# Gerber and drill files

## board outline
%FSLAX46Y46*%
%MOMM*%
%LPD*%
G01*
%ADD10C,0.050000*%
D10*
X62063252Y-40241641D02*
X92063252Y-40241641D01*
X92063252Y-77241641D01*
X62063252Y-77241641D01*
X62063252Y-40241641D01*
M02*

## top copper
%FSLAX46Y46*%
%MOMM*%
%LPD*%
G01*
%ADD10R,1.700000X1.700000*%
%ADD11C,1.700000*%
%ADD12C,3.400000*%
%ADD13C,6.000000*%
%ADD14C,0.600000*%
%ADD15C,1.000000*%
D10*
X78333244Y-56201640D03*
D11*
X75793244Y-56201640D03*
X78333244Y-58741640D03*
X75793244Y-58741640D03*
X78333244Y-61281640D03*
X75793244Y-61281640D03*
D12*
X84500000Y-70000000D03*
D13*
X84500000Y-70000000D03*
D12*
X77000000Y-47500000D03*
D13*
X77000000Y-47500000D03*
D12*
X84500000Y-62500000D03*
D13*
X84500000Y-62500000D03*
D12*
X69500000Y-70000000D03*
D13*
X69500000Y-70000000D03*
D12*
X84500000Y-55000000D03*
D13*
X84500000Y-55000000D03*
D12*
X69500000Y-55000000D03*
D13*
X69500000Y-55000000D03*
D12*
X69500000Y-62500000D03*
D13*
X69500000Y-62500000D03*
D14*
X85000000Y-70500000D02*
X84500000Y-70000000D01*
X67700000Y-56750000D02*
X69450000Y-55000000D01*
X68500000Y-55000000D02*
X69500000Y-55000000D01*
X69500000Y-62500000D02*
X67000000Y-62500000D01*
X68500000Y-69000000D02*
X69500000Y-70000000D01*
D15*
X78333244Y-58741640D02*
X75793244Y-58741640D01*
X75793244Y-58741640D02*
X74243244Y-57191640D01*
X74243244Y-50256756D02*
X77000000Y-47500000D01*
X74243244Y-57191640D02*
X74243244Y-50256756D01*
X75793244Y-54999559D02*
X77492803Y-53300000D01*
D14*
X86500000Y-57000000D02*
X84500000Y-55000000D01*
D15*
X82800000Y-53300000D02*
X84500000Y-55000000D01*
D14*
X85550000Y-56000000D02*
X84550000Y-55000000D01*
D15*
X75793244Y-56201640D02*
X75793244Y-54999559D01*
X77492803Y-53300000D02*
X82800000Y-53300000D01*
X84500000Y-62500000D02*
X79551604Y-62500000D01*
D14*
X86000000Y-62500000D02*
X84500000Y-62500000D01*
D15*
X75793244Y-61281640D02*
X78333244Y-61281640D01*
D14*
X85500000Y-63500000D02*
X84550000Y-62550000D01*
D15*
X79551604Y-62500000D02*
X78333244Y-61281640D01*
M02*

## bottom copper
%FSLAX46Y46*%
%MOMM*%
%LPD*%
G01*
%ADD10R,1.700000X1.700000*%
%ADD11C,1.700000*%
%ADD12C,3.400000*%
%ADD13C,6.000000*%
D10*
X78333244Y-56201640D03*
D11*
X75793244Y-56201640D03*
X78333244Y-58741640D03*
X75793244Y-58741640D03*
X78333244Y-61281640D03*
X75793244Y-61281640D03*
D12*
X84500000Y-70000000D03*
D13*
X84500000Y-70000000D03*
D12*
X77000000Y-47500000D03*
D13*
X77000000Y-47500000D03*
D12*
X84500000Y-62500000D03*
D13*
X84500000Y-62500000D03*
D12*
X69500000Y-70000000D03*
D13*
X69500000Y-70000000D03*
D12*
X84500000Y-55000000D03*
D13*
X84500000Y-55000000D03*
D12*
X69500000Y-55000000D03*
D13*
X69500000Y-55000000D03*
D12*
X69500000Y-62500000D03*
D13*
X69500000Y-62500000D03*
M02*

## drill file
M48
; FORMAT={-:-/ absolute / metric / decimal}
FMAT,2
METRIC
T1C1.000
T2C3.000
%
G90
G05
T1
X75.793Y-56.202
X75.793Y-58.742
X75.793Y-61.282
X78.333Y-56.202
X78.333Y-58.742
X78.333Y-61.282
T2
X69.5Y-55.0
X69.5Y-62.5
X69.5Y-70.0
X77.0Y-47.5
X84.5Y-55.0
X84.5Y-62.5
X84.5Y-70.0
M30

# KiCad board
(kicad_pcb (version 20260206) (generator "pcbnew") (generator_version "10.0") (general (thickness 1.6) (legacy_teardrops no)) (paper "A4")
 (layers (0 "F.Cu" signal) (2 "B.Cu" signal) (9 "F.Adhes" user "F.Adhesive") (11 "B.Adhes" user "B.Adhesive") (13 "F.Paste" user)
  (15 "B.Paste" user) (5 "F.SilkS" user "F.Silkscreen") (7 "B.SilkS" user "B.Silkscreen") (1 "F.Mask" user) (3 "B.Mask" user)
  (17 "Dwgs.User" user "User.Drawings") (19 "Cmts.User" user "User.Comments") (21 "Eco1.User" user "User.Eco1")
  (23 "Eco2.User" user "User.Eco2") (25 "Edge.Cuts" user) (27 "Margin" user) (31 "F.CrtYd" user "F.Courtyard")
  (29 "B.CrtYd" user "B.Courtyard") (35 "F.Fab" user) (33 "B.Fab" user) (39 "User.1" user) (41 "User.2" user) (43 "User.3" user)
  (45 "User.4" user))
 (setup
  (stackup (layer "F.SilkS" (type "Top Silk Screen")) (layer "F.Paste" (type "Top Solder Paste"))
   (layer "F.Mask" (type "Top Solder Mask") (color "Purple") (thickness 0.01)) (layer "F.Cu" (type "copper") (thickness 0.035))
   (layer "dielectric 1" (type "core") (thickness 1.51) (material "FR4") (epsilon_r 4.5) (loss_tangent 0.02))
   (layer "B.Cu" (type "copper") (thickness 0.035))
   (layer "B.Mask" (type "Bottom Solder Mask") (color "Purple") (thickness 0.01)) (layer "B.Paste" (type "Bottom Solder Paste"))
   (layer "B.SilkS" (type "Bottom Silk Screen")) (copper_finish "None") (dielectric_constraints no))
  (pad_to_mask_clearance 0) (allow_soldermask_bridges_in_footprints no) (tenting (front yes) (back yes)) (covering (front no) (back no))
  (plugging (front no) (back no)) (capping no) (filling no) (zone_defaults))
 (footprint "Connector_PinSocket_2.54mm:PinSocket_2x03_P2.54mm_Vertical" (layer "F.Cu") (at 78.333244 56.20164)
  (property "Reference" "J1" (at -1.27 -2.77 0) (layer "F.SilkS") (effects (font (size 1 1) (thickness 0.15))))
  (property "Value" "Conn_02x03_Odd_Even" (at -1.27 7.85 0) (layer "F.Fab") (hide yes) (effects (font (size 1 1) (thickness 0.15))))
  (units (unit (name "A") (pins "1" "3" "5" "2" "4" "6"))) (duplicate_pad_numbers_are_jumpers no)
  (pad "1" thru_hole rect (at 0 0) (size 1.7 1.7) (drill 1) (layers "*.Cu" "*.Mask") (remove_unused_layers no)
   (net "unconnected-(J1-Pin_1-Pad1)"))
  (pad "2" thru_hole circle (at -2.54 0) (size 1.7 1.7) (drill 1) (layers "*.Cu" "*.Mask") (remove_unused_layers no) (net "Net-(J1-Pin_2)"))
  (pad "3" thru_hole circle (at 0 2.54) (size 1.7 1.7) (drill 1) (layers "*.Cu" "*.Mask") (remove_unused_layers no) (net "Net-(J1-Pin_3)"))
  (pad "4" thru_hole circle (at -2.54 2.54) (size 1.7 1.7) (drill 1) (layers "*.Cu" "*.Mask") (remove_unused_layers no)
   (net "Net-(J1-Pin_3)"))
  (pad "5" thru_hole circle (at 0 5.08) (size 1.7 1.7) (drill 1) (layers "*.Cu" "*.Mask") (remove_unused_layers no) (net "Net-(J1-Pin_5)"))
  (pad "6" thru_hole circle (at -2.54 5.08) (size 1.7 1.7) (drill 1) (layers "*.Cu" "*.Mask") (remove_unused_layers no)
   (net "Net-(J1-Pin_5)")))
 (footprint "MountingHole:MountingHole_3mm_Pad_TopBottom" (layer "F.Cu") (at 84.5 70)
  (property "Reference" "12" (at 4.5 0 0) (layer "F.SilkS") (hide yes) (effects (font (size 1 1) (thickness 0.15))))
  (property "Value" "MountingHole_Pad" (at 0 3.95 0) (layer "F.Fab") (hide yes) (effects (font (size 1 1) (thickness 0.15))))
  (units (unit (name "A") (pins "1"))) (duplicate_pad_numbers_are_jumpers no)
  (pad "1" thru_hole circle (at 0 0) (size 3.4 3.4) (drill 3) (layers "*.Cu" "*.Mask") (remove_unused_layers no)
   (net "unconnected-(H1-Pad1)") (zone_connect 2))
  (pad "1" connect circle (at 0 0) (size 6 6) (layers "F.Cu" "F.Mask") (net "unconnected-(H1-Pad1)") (zone_connect 2))
  (pad "1" connect circle (at 0 0) (size 6 6) (layers "B.Cu" "B.Mask") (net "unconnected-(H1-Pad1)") (zone_connect 2)))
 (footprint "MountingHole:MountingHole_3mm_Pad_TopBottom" (layer "F.Cu") (at 77 47.5)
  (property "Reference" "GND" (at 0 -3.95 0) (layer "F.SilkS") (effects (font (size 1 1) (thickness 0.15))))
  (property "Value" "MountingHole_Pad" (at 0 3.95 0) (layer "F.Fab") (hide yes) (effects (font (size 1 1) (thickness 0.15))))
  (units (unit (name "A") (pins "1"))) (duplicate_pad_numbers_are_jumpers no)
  (pad "1" thru_hole circle (at 0 0) (size 3.4 3.4) (drill 3) (layers "*.Cu" "*.Mask") (remove_unused_layers no) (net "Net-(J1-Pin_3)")
   (zone_connect 2))
  (pad "1" connect circle (at 0 0) (size 6 6) (layers "F.Cu" "F.Mask") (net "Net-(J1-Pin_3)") (zone_connect 2))
  (pad "1" connect circle (at 0 0) (size 6 6) (layers "B.Cu" "B.Mask") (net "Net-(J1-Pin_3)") (zone_connect 2)))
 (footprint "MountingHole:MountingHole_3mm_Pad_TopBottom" (layer "F.Cu") (at 84.5 62.5)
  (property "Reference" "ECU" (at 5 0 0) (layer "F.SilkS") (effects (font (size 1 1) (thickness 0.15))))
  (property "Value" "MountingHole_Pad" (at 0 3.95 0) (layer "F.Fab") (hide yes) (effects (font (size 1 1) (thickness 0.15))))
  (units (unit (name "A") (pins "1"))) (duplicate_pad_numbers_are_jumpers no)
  (pad "1" thru_hole circle (at 0 0) (size 3.4 3.4) (drill 3) (layers "*.Cu" "*.Mask") (remove_unused_layers no) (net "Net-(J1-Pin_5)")
   (zone_connect 2))
  (pad "1" connect circle (at 0 0) (size 6 6) (layers "F.Cu" "F.Mask") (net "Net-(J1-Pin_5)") (zone_connect 2))
  (pad "1" connect circle (at 0 0) (size 6 6) (layers "B.Cu" "B.Mask") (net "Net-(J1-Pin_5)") (zone_connect 2)))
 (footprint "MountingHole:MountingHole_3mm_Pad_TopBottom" (layer "F.Cu") (at 69.5 70)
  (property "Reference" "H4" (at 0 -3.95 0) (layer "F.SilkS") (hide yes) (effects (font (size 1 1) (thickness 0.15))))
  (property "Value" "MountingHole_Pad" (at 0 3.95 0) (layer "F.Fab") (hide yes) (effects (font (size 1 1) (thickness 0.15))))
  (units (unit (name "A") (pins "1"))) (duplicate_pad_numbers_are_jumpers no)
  (pad "1" thru_hole circle (at 0 0) (size 3.4 3.4) (drill 3) (layers "*.Cu" "*.Mask") (remove_unused_layers no)
   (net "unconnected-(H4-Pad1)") (zone_connect 2))
  (pad "1" connect circle (at 0 0) (size 6 6) (layers "F.Cu" "F.Mask") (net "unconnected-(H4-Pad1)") (zone_connect 2))
  (pad "1" connect circle (at 0 0) (size 6 6) (layers "B.Cu" "B.Mask") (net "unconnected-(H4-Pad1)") (zone_connect 2)))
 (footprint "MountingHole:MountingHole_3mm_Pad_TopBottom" (layer "F.Cu") (at 84.5 55)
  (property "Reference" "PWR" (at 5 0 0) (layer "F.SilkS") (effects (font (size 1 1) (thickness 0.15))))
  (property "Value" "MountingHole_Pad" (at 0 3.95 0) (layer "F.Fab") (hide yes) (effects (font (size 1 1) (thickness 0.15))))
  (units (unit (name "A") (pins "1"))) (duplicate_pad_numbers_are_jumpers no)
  (pad "1" thru_hole circle (at 0 0) (size 3.4 3.4) (drill 3) (layers "*.Cu" "*.Mask") (remove_unused_layers no) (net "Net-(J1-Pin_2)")
   (zone_connect 2))
  (pad "1" connect circle (at 0 0) (size 6 6) (layers "F.Cu" "F.Mask") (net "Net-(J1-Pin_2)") (zone_connect 2))
  (pad "1" connect circle (at 0 0) (size 6 6) (layers "B.Cu" "B.Mask") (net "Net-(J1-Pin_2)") (zone_connect 2)))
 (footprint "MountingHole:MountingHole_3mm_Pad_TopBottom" (layer "F.Cu") (at 69.5 55)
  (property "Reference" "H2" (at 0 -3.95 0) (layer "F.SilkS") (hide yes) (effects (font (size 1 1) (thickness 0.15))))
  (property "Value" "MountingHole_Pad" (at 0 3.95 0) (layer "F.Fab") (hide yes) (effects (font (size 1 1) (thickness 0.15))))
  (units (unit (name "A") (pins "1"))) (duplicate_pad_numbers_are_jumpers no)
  (pad "1" thru_hole circle (at 0 0) (size 3.4 3.4) (drill 3) (layers "*.Cu" "*.Mask") (remove_unused_layers no)
   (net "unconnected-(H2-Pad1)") (zone_connect 2))
  (pad "1" connect circle (at 0 0) (size 6 6) (layers "F.Cu" "F.Mask") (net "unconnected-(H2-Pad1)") (zone_connect 2))
  (pad "1" connect circle (at 0 0) (size 6 6) (layers "B.Cu" "B.Mask") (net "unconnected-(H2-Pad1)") (zone_connect 2)))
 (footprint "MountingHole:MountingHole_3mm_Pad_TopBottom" (layer "F.Cu") (at 69.5 62.5)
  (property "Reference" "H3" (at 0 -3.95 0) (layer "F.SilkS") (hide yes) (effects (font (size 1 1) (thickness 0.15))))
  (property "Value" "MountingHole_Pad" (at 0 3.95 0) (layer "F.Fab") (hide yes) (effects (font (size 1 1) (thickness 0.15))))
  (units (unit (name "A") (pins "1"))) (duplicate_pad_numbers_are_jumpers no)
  (pad "1" thru_hole circle (at 0 0) (size 3.4 3.4) (drill 3) (layers "*.Cu" "*.Mask") (remove_unused_layers no)
   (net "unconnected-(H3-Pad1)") (zone_connect 2))
  (pad "1" connect circle (at 0 0) (size 6 6) (layers "F.Cu" "F.Mask") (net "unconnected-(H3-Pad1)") (zone_connect 2))
  (pad "1" connect circle (at 0 0) (size 6 6) (layers "B.Cu" "B.Mask") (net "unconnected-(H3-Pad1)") (zone_connect 2)))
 (gr_rect (start 62.063252 40.241641) (end 92.063252 77.241641) (stroke (width 0.05) (type default)) (fill no) (layer "Edge.Cuts"))
 (segment (start 85 70.5) (end 84.5 70) (width 0.6) (layer "F.Cu") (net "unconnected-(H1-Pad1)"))
 (segment (start 67.7 56.75) (end 69.45 55) (width 0.6) (layer "F.Cu") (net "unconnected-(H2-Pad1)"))
 (segment (start 68.5 55) (end 69.5 55) (width 0.6) (layer "F.Cu") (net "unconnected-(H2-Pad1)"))
 (segment (start 69.5 62.5) (end 67 62.5) (width 0.6) (layer "F.Cu") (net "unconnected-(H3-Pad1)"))
 (segment (start 68.5 69) (end 69.5 70) (width 0.6) (layer "F.Cu") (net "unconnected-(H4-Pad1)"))
 (segment (start 78.333244 58.74164) (end 75.793244 58.74164) (width 1) (layer "F.Cu") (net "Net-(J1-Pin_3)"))
 (segment (start 75.793244 58.74164) (end 74.243244 57.19164) (width 1) (layer "F.Cu") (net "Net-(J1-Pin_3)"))
 (segment (start 74.243244 50.256756) (end 77 47.5) (width 1) (layer "F.Cu") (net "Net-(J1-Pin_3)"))
 (segment (start 74.243244 57.19164) (end 74.243244 50.256756) (width 1) (layer "F.Cu") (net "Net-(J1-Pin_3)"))
 (segment (start 75.793244 54.999559) (end 77.492803 53.3) (width 1) (layer "F.Cu") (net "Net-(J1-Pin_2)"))
 (segment (start 86.5 57) (end 84.5 55) (width 0.6) (layer "F.Cu") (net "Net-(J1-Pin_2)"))
 (segment (start 82.8 53.3) (end 84.5 55) (width 1) (layer "F.Cu") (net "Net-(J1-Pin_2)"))
 (segment (start 85.55 56) (end 84.55 55) (width 0.6) (layer "F.Cu") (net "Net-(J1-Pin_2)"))
 (segment (start 75.793244 56.20164) (end 75.793244 54.999559) (width 1) (layer "F.Cu") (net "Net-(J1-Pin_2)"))
 (segment (start 77.492803 53.3) (end 82.8 53.3) (width 1) (layer "F.Cu") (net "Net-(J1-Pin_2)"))
 (segment (start 84.5 62.5) (end 79.551604 62.5) (width 1) (layer "F.Cu") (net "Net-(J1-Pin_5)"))
 (segment (start 86 62.5) (end 84.5 62.5) (width 0.6) (layer "F.Cu") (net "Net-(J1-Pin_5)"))
 (segment (start 75.793244 61.28164) (end 78.333244 61.28164) (width 1) (layer "F.Cu") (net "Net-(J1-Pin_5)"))
 (segment (start 85.5 63.5) (end 84.55 62.55) (width 0.6) (layer "F.Cu") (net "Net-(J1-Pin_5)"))
 (segment (start 79.551604 62.5) (end 78.333244 61.28164) (width 1) (layer "F.Cu") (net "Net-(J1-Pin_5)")))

